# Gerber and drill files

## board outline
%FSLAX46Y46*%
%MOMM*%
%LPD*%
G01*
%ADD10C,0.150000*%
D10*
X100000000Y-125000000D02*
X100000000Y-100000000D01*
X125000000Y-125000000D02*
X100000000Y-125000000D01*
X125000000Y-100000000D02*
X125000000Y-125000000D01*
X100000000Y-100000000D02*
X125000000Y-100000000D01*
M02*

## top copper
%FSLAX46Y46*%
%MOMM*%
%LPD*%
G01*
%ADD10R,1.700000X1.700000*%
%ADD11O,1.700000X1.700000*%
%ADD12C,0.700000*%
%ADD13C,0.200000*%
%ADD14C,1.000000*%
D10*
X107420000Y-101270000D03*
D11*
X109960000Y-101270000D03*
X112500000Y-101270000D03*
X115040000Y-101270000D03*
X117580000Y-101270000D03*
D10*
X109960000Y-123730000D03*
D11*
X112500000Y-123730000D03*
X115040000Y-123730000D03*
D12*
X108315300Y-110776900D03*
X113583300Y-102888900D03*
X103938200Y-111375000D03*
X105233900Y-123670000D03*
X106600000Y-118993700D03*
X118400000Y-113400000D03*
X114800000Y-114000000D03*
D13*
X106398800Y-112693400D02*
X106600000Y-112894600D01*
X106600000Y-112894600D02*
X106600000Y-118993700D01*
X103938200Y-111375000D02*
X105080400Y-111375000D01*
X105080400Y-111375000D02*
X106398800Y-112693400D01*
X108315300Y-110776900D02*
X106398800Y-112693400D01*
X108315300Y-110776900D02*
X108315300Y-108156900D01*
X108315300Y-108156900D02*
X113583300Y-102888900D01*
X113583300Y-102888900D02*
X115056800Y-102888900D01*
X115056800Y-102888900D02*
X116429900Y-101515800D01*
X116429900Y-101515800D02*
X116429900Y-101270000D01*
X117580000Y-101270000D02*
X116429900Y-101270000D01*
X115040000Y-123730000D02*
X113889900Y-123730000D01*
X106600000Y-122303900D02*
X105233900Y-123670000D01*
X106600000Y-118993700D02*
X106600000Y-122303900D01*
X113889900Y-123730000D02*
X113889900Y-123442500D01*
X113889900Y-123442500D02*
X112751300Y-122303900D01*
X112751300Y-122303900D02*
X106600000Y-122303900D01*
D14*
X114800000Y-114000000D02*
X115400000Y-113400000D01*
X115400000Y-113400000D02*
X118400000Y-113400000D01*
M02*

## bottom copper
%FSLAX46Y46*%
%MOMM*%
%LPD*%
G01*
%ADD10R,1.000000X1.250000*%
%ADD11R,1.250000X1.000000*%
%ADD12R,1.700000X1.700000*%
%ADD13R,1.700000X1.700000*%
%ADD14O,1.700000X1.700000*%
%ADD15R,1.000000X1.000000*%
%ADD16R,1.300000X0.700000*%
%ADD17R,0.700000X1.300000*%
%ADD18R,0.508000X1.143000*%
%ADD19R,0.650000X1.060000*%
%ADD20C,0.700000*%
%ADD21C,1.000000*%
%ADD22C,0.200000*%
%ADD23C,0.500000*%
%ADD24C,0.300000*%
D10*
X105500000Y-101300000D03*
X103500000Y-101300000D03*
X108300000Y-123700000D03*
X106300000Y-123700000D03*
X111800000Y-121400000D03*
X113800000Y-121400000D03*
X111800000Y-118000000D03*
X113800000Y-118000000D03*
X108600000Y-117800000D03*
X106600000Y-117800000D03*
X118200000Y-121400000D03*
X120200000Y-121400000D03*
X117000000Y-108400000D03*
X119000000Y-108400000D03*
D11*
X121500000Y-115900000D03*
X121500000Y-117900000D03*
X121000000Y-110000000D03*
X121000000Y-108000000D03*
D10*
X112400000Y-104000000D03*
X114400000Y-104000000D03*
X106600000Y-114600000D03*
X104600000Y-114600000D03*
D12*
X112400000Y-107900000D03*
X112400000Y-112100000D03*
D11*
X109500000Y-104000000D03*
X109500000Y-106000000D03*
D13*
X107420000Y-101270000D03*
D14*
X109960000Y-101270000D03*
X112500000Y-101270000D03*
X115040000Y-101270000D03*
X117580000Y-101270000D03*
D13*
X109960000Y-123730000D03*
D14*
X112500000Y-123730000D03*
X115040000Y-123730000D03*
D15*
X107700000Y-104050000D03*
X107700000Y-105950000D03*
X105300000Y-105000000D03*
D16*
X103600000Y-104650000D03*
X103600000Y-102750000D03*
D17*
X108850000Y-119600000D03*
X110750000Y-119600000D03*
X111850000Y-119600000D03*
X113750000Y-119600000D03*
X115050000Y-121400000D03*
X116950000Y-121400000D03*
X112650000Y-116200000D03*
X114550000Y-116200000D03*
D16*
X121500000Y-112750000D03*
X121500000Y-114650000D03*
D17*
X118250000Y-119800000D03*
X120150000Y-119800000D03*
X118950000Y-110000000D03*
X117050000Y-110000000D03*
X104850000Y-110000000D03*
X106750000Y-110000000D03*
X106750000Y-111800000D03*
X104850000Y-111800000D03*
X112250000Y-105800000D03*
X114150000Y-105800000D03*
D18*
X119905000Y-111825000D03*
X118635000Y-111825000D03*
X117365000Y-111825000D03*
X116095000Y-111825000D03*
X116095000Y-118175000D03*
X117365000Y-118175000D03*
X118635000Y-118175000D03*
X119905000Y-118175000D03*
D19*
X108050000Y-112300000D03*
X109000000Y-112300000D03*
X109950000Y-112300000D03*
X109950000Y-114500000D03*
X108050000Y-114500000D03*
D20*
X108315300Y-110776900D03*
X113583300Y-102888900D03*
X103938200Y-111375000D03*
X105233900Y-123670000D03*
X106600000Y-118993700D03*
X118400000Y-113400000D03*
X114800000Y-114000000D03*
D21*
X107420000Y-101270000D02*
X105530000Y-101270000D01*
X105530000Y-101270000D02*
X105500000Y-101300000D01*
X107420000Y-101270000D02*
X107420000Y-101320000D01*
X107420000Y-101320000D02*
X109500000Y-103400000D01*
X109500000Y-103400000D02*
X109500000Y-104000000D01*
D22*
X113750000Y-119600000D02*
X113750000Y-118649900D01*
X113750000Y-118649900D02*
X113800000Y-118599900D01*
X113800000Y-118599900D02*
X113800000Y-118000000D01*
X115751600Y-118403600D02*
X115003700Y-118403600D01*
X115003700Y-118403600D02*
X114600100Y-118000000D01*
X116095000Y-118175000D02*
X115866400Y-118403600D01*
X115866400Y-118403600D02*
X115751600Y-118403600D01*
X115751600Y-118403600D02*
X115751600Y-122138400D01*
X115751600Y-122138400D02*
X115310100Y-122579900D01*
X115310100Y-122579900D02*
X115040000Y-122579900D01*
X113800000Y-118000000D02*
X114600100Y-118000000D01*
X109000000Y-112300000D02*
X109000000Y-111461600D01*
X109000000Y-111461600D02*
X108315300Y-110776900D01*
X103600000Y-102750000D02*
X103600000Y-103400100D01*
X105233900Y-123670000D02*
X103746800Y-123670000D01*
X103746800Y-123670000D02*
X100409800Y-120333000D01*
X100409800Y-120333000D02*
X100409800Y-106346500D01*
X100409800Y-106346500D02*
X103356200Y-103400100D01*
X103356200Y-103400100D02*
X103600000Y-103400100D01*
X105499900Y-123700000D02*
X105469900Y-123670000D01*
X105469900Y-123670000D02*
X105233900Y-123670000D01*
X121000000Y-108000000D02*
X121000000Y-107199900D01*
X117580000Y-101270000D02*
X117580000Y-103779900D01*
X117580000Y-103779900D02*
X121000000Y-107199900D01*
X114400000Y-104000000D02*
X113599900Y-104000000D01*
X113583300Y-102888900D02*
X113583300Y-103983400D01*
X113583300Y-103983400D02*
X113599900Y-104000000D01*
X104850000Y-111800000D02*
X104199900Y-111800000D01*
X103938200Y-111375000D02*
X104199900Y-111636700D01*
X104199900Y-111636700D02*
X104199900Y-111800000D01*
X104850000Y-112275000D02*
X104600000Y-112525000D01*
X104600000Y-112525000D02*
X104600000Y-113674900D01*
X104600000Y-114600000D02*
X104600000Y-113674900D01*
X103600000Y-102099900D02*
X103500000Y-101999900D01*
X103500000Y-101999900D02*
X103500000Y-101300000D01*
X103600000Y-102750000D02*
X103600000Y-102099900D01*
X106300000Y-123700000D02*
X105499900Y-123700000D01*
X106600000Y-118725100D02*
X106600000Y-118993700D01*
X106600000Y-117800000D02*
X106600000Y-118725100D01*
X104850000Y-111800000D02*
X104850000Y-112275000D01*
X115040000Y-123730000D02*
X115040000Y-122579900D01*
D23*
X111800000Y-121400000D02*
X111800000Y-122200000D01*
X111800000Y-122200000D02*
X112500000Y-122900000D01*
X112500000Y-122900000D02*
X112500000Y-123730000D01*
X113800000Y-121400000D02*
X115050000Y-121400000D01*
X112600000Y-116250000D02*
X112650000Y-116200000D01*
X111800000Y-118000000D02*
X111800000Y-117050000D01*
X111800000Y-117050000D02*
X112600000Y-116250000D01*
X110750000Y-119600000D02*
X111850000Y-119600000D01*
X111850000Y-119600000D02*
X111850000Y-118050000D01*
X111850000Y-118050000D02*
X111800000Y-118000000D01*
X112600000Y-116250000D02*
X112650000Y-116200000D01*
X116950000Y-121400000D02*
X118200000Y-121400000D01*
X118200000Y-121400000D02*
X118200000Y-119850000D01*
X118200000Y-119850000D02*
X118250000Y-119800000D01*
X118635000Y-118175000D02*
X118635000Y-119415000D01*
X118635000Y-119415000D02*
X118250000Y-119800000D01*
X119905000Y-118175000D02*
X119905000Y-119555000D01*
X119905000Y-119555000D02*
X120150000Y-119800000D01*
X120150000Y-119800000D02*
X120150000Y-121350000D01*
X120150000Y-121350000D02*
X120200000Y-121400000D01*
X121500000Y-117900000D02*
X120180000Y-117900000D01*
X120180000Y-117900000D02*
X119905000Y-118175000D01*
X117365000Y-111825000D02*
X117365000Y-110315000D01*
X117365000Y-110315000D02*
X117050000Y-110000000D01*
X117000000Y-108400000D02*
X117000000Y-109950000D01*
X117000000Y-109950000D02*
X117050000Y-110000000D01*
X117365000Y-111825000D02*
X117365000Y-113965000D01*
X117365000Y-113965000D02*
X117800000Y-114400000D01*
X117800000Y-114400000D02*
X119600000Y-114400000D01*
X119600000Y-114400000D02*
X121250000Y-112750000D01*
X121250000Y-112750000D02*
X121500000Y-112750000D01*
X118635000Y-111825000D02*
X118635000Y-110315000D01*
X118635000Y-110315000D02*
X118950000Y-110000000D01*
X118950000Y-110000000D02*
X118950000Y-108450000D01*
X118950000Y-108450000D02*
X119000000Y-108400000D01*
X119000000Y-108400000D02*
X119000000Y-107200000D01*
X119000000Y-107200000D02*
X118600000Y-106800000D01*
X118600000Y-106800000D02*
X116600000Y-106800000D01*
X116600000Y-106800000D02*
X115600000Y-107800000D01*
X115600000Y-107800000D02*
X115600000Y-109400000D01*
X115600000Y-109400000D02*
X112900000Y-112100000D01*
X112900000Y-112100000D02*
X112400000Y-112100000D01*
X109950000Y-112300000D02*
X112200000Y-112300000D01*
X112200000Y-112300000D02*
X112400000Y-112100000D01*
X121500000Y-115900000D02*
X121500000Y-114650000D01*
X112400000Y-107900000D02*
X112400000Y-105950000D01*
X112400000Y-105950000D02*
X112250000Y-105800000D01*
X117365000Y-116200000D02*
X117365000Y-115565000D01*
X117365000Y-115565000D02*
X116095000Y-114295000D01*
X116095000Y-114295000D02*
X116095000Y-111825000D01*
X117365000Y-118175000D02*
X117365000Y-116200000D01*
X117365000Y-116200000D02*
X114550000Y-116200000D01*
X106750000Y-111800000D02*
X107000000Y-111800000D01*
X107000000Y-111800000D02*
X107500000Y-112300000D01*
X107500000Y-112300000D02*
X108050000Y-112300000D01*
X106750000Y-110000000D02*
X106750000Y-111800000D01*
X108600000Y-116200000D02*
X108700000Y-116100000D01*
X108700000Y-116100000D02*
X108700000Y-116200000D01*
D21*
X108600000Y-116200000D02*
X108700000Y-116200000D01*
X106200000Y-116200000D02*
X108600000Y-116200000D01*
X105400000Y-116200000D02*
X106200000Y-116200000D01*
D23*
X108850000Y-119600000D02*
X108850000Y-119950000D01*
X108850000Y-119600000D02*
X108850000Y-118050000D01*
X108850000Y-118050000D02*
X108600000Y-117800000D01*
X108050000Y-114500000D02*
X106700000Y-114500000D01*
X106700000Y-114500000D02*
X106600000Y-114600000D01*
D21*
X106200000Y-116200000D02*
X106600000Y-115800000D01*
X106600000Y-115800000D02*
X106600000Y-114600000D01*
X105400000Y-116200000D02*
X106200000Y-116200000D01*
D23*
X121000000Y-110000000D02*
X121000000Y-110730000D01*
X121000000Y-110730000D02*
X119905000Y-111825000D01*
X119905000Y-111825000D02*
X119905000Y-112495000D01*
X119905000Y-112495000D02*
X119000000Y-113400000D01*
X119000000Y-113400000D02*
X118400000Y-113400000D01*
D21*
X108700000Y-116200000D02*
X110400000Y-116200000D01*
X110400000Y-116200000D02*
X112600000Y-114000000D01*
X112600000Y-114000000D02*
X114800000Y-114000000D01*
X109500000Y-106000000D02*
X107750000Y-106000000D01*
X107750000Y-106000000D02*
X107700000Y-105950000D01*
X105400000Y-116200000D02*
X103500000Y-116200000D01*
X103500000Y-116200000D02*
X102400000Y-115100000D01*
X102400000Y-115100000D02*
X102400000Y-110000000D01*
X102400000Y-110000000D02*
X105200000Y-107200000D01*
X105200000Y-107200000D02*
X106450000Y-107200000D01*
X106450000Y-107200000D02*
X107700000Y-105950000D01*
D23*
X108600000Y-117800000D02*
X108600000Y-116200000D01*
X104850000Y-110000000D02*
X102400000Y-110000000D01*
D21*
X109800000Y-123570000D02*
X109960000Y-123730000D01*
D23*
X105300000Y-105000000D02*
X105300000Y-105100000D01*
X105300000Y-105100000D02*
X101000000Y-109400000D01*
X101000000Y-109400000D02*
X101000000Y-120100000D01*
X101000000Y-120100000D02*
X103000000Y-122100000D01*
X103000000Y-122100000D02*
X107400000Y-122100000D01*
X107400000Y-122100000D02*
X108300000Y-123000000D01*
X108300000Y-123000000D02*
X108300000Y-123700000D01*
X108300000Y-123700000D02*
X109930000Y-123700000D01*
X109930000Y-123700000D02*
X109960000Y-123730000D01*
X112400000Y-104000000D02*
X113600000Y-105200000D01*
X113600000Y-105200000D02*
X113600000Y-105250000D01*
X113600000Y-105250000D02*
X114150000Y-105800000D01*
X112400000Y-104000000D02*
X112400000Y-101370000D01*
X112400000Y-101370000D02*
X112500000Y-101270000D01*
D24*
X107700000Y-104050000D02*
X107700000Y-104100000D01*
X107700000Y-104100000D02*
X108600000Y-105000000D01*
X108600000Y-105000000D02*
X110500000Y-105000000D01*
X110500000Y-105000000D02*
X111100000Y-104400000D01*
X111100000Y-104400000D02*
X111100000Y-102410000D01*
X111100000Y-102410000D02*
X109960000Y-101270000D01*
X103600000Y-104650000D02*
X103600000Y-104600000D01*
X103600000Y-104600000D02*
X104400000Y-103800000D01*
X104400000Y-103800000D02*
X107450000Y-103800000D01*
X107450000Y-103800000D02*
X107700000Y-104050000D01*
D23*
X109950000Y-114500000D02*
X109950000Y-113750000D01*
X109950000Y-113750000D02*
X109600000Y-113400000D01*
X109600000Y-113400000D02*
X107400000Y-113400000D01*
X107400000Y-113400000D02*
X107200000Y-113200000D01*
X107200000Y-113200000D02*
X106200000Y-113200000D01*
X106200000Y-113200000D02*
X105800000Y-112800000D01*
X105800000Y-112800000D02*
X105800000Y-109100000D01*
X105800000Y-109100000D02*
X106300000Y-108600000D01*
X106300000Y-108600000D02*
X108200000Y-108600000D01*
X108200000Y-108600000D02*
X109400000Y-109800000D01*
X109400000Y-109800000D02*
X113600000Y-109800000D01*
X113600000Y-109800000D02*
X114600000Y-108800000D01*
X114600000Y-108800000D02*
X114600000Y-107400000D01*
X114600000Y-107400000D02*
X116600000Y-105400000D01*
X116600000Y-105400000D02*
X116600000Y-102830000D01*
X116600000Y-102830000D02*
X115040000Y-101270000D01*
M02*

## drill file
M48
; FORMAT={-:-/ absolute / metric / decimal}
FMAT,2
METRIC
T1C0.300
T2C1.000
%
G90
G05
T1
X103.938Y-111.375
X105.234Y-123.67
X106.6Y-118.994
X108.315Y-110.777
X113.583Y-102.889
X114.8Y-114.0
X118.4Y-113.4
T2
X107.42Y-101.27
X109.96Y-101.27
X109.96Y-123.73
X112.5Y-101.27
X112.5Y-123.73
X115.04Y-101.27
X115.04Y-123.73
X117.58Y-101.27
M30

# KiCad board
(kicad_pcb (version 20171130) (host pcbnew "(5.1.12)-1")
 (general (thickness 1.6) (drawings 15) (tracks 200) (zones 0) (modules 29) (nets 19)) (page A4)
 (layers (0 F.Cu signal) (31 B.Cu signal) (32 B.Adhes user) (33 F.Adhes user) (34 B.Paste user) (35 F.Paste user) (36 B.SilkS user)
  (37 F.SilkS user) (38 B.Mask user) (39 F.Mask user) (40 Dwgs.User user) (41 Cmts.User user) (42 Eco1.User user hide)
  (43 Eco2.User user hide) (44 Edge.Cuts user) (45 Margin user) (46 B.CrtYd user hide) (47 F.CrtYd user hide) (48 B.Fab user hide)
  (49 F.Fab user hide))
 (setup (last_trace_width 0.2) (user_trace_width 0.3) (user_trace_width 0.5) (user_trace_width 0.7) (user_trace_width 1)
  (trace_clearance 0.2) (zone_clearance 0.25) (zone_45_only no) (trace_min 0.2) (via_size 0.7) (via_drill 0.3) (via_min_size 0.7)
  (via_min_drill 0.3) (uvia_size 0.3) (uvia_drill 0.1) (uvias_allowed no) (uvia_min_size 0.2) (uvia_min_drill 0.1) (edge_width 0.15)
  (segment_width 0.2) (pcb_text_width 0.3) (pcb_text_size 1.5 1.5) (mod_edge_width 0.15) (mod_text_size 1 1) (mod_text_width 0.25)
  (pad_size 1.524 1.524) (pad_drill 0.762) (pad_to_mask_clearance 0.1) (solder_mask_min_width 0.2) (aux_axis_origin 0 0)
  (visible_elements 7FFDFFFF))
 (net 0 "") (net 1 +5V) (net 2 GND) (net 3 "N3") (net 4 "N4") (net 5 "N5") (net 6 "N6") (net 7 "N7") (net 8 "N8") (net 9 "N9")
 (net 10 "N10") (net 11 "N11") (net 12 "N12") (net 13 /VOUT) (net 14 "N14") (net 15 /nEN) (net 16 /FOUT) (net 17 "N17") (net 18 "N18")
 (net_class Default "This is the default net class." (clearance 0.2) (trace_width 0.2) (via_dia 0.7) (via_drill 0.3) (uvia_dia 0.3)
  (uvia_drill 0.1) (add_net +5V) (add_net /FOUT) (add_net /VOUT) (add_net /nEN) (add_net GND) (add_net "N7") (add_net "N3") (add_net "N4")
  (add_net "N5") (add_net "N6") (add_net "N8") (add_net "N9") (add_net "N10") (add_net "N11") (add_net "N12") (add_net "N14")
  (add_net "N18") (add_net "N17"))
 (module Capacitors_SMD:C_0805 (layer B.Cu) (at 104.5 101.3 180)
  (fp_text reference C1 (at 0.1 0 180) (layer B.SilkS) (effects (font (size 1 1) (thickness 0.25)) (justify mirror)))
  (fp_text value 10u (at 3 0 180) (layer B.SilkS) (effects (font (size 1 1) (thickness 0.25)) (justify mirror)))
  (pad 1 smd rect (at -1 0 180) (size 1 1.25) (layers B.Cu B.Paste B.Mask) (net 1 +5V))
  (pad 2 smd rect (at 1 0 180) (size 1 1.25) (layers B.Cu B.Paste B.Mask) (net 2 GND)))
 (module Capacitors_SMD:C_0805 (layer B.Cu) (at 107.3 123.7 180)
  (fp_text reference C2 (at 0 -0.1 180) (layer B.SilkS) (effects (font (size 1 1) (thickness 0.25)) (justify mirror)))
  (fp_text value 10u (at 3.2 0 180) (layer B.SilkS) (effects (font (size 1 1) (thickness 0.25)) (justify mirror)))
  (pad 1 smd rect (at -1 0 180) (size 1 1.25) (layers B.Cu B.Paste B.Mask) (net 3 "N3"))
  (pad 2 smd rect (at 1 0 180) (size 1 1.25) (layers B.Cu B.Paste B.Mask) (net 2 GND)))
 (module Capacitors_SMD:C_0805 (layer B.Cu) (at 112.8 121.4)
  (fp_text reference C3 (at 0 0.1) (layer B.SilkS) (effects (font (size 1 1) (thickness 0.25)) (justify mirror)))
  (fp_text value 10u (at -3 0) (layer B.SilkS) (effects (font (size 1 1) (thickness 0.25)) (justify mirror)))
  (pad 1 smd rect (at -1 0) (size 1 1.25) (layers B.Cu B.Paste B.Mask) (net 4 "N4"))
  (pad 2 smd rect (at 1 0) (size 1 1.25) (layers B.Cu B.Paste B.Mask) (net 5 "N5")))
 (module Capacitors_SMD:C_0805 (layer B.Cu) (at 112.8 118)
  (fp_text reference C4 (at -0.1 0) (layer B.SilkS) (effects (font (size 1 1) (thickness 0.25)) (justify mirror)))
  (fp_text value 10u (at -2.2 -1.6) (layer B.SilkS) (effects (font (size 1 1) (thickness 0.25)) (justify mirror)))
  (pad 1 smd rect (at -1 0) (size 1 1.25) (layers B.Cu B.Paste B.Mask) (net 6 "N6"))
  (pad 2 smd rect (at 1 0) (size 1 1.25) (layers B.Cu B.Paste B.Mask) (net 2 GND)))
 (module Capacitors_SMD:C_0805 (layer B.Cu) (at 107.6 117.8 180)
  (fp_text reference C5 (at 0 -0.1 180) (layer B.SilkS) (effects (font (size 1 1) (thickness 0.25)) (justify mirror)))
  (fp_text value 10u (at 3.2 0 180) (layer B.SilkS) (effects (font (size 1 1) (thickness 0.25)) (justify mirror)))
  (pad 1 smd rect (at -1 0 180) (size 1 1.25) (layers B.Cu B.Paste B.Mask) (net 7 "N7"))
  (pad 2 smd rect (at 1 0 180) (size 1 1.25) (layers B.Cu B.Paste B.Mask) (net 2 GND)))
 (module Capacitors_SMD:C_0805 (layer B.Cu) (at 119.2 121.4)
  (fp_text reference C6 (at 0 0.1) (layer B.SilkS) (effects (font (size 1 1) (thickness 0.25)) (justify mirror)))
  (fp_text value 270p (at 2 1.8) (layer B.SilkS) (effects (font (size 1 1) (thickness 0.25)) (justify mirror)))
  (pad 1 smd rect (at -1 0) (size 1 1.25) (layers B.Cu B.Paste B.Mask) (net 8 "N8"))
  (pad 2 smd rect (at 1 0) (size 1 1.25) (layers B.Cu B.Paste B.Mask) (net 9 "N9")))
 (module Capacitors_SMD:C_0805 (layer B.Cu) (at 118 108.4)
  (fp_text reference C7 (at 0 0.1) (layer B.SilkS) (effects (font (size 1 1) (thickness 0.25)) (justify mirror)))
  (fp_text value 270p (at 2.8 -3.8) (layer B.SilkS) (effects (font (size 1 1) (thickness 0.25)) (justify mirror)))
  (pad 1 smd rect (at -1 0) (size 1 1.25) (layers B.Cu B.Paste B.Mask) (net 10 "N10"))
  (pad 2 smd rect (at 1 0) (size 1 1.25) (layers B.Cu B.Paste B.Mask) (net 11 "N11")))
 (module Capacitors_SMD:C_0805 (layer B.Cu) (at 121.5 116.9 270)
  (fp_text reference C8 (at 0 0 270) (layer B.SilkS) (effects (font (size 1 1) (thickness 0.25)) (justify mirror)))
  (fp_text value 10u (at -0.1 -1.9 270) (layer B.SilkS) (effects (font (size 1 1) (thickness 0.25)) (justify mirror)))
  (pad 1 smd rect (at -1 0 270) (size 1 1.25) (layers B.Cu B.Paste B.Mask) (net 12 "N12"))
  (pad 2 smd rect (at 1 0 270) (size 1 1.25) (layers B.Cu B.Paste B.Mask) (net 9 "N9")))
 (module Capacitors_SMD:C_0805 (layer B.Cu) (at 121 109 90)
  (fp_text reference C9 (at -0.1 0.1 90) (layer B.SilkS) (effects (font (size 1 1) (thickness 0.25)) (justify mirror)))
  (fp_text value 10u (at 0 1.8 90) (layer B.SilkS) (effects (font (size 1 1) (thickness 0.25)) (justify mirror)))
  (pad 1 smd rect (at -1 0 90) (size 1 1.25) (layers B.Cu B.Paste B.Mask) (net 7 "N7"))
  (pad 2 smd rect (at 1 0 90) (size 1 1.25) (layers B.Cu B.Paste B.Mask) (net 2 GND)))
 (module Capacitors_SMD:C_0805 (layer B.Cu) (at 113.4 104)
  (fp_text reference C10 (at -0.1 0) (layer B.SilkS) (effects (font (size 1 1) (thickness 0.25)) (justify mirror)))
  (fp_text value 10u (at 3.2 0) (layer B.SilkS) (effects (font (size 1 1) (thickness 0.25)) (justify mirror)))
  (pad 1 smd rect (at -1 0) (size 1 1.25) (layers B.Cu B.Paste B.Mask) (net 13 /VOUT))
  (pad 2 smd rect (at 1 0) (size 1 1.25) (layers B.Cu B.Paste B.Mask) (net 2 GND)))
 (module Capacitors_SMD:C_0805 (layer B.Cu) (at 105.6 114.6 180)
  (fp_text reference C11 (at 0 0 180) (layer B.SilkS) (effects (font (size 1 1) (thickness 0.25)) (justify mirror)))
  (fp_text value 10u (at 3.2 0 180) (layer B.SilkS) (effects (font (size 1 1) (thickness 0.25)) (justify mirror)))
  (pad 1 smd rect (at -1 0 180) (size 1 1.25) (layers B.Cu B.Paste B.Mask) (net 7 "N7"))
  (pad 2 smd rect (at 1 0 180) (size 1 1.25) (layers B.Cu B.Paste B.Mask) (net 2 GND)))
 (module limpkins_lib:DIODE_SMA (layer B.Cu) (at 112.4 110 270)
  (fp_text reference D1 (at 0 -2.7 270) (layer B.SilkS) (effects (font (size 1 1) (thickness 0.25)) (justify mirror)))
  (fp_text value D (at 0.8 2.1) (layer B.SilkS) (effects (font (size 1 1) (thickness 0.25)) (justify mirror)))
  (pad 1 smd rect (at -2.1 0 270) (size 1.7 1.7) (layers B.Cu B.Paste B.Mask) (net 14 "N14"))
  (pad 2 smd rect (at 2.1 0 270) (size 1.7 1.7) (layers B.Cu B.Paste B.Mask) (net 11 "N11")))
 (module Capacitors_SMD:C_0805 (layer B.Cu) (at 109.5 105 270)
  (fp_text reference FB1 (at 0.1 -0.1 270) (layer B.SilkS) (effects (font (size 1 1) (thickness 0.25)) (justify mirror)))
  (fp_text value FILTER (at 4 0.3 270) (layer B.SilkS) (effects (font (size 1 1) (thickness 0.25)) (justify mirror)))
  (pad 1 smd rect (at -1 0 270) (size 1 1.25) (layers B.Cu B.Paste B.Mask) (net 1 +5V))
  (pad 2 smd rect (at 1 0 270) (size 1 1.25) (layers B.Cu B.Paste B.Mask) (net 7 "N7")))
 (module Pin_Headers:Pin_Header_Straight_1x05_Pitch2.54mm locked (layer F.Cu) (at 107.42 101.27 90)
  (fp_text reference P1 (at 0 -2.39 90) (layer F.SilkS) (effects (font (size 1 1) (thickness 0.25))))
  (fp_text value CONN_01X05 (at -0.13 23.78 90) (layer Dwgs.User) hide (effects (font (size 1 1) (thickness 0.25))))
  (pad 1 thru_hole rect (at 0 0 90) (size 1.7 1.7) (drill 1) (layers *.Cu *.Mask) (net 1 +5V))
  (pad 2 thru_hole oval (at 0 2.54 90) (size 1.7 1.7) (drill 1) (layers *.Cu *.Mask) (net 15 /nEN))
  (pad 3 thru_hole oval (at 0 5.08 90) (size 1.7 1.7) (drill 1) (layers *.Cu *.Mask) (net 13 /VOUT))
  (pad 4 thru_hole oval (at 0 7.62 90) (size 1.7 1.7) (drill 1) (layers *.Cu *.Mask) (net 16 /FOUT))
  (pad 5 thru_hole oval (at 0 10.16 90) (size 1.7 1.7) (drill 1) (layers *.Cu *.Mask) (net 2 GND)))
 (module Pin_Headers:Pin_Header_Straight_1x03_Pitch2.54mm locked (layer F.Cu) (at 109.96 123.73 90)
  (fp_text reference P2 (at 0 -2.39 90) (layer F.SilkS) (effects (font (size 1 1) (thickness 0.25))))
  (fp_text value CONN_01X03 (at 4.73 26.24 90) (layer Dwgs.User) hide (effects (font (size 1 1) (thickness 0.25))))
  (pad 1 thru_hole rect (at 0 0 90) (size 1.7 1.7) (drill 1) (layers *.Cu *.Mask) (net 3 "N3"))
  (pad 2 thru_hole oval (at 0 2.54 90) (size 1.7 1.7) (drill 1) (layers *.Cu *.Mask) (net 4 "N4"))
  (pad 3 thru_hole oval (at 0 5.08 90) (size 1.7 1.7) (drill 1) (layers *.Cu *.Mask) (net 2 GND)))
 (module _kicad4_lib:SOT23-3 (layer B.Cu) (at 106.5 105 270)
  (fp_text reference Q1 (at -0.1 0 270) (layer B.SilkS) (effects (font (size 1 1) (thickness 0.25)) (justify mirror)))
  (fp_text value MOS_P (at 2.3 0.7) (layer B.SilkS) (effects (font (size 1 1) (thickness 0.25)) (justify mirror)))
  (pad 1 smd rect (at -0.95 -1.2 270) (size 1 1) (layers B.Cu B.Paste B.Mask) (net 15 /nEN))
  (pad 2 smd rect (at 0.95 -1.2 270) (size 1 1) (layers B.Cu B.Paste B.Mask) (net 7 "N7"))
  (pad 3 smd rect (at 0 1.2 270) (size 1 1) (layers B.Cu B.Paste B.Mask) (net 3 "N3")))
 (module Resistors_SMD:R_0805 (layer B.Cu) (at 103.6 103.7 90)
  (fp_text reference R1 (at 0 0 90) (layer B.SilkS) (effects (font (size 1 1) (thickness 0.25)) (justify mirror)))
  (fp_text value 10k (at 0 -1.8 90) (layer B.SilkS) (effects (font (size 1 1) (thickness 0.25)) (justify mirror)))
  (pad 1 smd rect (at -0.95 0 90) (size 0.7 1.3) (layers B.Cu B.Paste B.Mask) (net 15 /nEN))
  (pad 2 smd rect (at 0.95 0 90) (size 0.7 1.3) (layers B.Cu B.Paste B.Mask) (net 2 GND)))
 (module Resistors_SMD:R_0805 (layer B.Cu) (at 109.8 119.6)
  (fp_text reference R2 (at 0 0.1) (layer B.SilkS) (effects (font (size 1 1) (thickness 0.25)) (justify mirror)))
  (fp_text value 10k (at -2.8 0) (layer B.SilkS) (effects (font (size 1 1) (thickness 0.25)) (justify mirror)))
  (pad 1 smd rect (at -0.95 0) (size 0.7 1.3) (layers B.Cu B.Paste B.Mask) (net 7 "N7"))
  (pad 2 smd rect (at 0.95 0) (size 0.7 1.3) (layers B.Cu B.Paste B.Mask) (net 6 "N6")))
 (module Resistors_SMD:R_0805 (layer B.Cu) (at 112.8 119.6)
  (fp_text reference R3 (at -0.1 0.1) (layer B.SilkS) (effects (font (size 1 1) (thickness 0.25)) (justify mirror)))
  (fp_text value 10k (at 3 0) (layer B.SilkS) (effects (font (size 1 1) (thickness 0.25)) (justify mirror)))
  (pad 1 smd rect (at -0.95 0) (size 0.7 1.3) (layers B.Cu B.Paste B.Mask) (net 6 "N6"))
  (pad 2 smd rect (at 0.95 0) (size 0.7 1.3) (layers B.Cu B.Paste B.Mask) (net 2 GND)))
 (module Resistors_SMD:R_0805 (layer B.Cu) (at 116 121.4)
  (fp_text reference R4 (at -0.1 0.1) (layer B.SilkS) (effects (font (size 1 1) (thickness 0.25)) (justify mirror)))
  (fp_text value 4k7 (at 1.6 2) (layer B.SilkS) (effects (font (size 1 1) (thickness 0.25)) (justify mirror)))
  (pad 1 smd rect (at -0.95 0) (size 0.7 1.3) (layers B.Cu B.Paste B.Mask) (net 5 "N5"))
  (pad 2 smd rect (at 0.95 0) (size 0.7 1.3) (layers B.Cu B.Paste B.Mask) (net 8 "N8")))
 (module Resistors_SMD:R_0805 (layer B.Cu) (at 113.6 116.2)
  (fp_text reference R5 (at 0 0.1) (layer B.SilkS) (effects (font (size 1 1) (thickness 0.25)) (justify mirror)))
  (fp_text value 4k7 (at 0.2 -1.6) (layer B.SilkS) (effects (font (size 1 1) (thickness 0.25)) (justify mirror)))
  (pad 1 smd rect (at -0.95 0) (size 0.7 1.3) (layers B.Cu B.Paste B.Mask) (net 6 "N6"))
  (pad 2 smd rect (at 0.95 0) (size 0.7 1.3) (layers B.Cu B.Paste B.Mask) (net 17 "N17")))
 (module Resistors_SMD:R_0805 (layer B.Cu) (at 121.5 113.7 270)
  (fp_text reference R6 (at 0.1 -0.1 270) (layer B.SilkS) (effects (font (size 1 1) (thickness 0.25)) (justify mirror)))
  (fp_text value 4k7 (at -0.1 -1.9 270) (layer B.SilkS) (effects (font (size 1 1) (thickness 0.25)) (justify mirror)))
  (pad 1 smd rect (at -0.95 0 270) (size 0.7 1.3) (layers B.Cu B.Paste B.Mask) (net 10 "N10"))
  (pad 2 smd rect (at 0.95 0 270) (size 0.7 1.3) (layers B.Cu B.Paste B.Mask) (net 12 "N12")))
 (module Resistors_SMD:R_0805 (layer B.Cu) (at 119.2 119.8)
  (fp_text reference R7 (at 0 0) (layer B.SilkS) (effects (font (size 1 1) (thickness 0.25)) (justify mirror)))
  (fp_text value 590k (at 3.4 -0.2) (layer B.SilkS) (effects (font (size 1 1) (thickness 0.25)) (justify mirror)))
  (pad 1 smd rect (at -0.95 0) (size 0.7 1.3) (layers B.Cu B.Paste B.Mask) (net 8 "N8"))
  (pad 2 smd rect (at 0.95 0) (size 0.7 1.3) (layers B.Cu B.Paste B.Mask) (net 9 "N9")))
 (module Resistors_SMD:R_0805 (layer B.Cu) (at 118 110 180)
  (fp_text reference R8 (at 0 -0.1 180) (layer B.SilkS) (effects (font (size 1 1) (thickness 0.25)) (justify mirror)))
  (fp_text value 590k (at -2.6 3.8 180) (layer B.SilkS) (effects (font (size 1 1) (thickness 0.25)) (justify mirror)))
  (pad 1 smd rect (at -0.95 0 180) (size 0.7 1.3) (layers B.Cu B.Paste B.Mask) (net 11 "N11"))
  (pad 2 smd rect (at 0.95 0 180) (size 0.7 1.3) (layers B.Cu B.Paste B.Mask) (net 10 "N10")))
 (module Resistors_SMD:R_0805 (layer B.Cu) (at 105.8 110)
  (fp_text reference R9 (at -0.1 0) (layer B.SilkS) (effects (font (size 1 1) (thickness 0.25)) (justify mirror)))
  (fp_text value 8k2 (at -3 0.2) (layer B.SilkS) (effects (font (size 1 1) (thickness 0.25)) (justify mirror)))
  (pad 1 smd rect (at -0.95 0) (size 0.7 1.3) (layers B.Cu B.Paste B.Mask) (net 7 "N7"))
  (pad 2 smd rect (at 0.95 0) (size 0.7 1.3) (layers B.Cu B.Paste B.Mask) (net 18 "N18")))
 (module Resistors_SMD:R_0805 (layer B.Cu) (at 105.8 111.8 180)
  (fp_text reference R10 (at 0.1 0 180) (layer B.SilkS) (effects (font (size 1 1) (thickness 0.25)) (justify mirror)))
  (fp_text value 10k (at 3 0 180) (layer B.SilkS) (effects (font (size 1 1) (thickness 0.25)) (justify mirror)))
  (pad 1 smd rect (at -0.95 0 180) (size 0.7 1.3) (layers B.Cu B.Paste B.Mask) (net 18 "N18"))
  (pad 2 smd rect (at 0.95 0 180) (size 0.7 1.3) (layers B.Cu B.Paste B.Mask) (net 2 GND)))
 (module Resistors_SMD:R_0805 (layer B.Cu) (at 113.2 105.8)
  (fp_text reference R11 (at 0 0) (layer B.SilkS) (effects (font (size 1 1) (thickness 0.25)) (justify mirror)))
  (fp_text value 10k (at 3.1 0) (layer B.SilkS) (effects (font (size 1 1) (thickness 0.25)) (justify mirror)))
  (pad 1 smd rect (at -0.95 0) (size 0.7 1.3) (layers B.Cu B.Paste B.Mask) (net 14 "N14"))
  (pad 2 smd rect (at 0.95 0) (size 0.7 1.3) (layers B.Cu B.Paste B.Mask) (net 13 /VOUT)))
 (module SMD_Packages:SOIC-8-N (layer B.Cu) (at 118 115 180)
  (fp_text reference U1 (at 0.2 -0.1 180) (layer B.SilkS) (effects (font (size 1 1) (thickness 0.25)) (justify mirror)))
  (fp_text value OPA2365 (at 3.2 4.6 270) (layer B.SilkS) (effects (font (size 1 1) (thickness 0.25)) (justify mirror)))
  (pad 8 smd rect (at -1.905 3.175 180) (size 0.508 1.143) (layers B.Cu B.Paste B.Mask) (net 7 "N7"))
  (pad 7 smd rect (at -0.635 3.175 180) (size 0.508 1.143) (layers B.Cu B.Paste B.Mask) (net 11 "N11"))
  (pad 6 smd rect (at 0.635 3.175 180) (size 0.508 1.143) (layers B.Cu B.Paste B.Mask) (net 10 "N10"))
  (pad 5 smd rect (at 1.905 3.175 180) (size 0.508 1.143) (layers B.Cu B.Paste B.Mask) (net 17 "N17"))
  (pad 4 smd rect (at 1.905 -3.175 180) (size 0.508 1.143) (layers B.Cu B.Paste B.Mask) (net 2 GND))
  (pad 3 smd rect (at 0.635 -3.175 180) (size 0.508 1.143) (layers B.Cu B.Paste B.Mask) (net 17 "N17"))
  (pad 2 smd rect (at -0.635 -3.175 180) (size 0.508 1.143) (layers B.Cu B.Paste B.Mask) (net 8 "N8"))
  (pad 1 smd rect (at -1.905 -3.175 180) (size 0.508 1.143) (layers B.Cu B.Paste B.Mask) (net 9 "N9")))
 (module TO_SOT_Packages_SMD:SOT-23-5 (layer B.Cu) (at 109 113.4 270)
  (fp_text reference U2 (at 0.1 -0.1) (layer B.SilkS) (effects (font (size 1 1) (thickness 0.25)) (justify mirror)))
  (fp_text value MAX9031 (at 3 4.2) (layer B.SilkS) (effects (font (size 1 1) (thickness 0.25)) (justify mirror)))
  (pad 1 smd rect (at -1.1 0.95 270) (size 1.06 0.65) (layers B.Cu B.Paste B.Mask) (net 18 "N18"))
  (pad 2 smd rect (at -1.1 0 270) (size 1.06 0.65) (layers B.Cu B.Paste B.Mask) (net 2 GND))
  (pad 3 smd rect (at -1.1 -0.95 270) (size 1.06 0.65) (layers B.Cu B.Paste B.Mask) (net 11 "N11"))
  (pad 4 smd rect (at 1.1 -0.95 270) (size 1.06 0.65) (layers B.Cu B.Paste B.Mask) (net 16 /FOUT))
  (pad 5 smd rect (at 1.1 0.95 270) (size 1.06 0.65) (layers B.Cu B.Paste B.Mask) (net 7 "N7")))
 (gr_line (start 100 125) (end 100 100) (angle 90) (layer Edge.Cuts) (width 0.15))
 (gr_line (start 125 125) (end 100 125) (angle 90) (layer Edge.Cuts) (width 0.15))
 (gr_line (start 125 100) (end 125 125) (angle 90) (layer Edge.Cuts) (width 0.15))
 (gr_line (start 100 100) (end 125 100) (angle 90) (layer Edge.Cuts) (width 0.15))
 (segment (start 107.42 101.27) (end 105.53 101.27) (width 1) (layer B.Cu) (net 1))
 (segment (start 105.53 101.27) (end 105.5 101.3) (width 1) (layer B.Cu) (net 1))
 (segment (start 107.42 101.27) (end 107.42 101.32) (width 1) (layer B.Cu) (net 1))
 (segment (start 107.42 101.32) (end 109.5 103.4) (width 1) (layer B.Cu) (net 1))
 (segment (start 109.5 103.4) (end 109.5 104) (width 1) (layer B.Cu) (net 1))
 (segment (start 113.75 119.6) (end 113.75 118.6499) (width 0.2) (layer B.Cu) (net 2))
 (segment (start 113.75 118.6499) (end 113.8 118.5999) (width 0.2) (layer B.Cu) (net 2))
 (segment (start 113.8 118.5999) (end 113.8 118) (width 0.2) (layer B.Cu) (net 2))
 (segment (start 115.7516 118.4036) (end 115.0037 118.4036) (width 0.2) (layer B.Cu) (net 2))
 (segment (start 115.0037 118.4036) (end 114.6001 118) (width 0.2) (layer B.Cu) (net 2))
 (segment (start 116.095 118.175) (end 115.8664 118.4036) (width 0.2) (layer B.Cu) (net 2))
 (segment (start 115.8664 118.4036) (end 115.7516 118.4036) (width 0.2) (layer B.Cu) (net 2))
 (segment (start 115.7516 118.4036) (end 115.7516 122.1384) (width 0.2) (layer B.Cu) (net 2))
 (segment (start 115.7516 122.1384) (end 115.3101 122.5799) (width 0.2) (layer B.Cu) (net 2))
 (segment (start 115.3101 122.5799) (end 115.04 122.5799) (width 0.2) (layer B.Cu) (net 2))
 (segment (start 113.8 118) (end 114.6001 118) (width 0.2) (layer B.Cu) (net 2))
 (segment (start 109 112.3) (end 109 111.4616) (width 0.2) (layer B.Cu) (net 2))
 (segment (start 109 111.4616) (end 108.3153 110.7769) (width 0.2) (layer B.Cu) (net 2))
 (segment (start 106.3988 112.6934) (end 106.6 112.8946) (width 0.2) (layer F.Cu) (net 2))
 (segment (start 106.6 112.8946) (end 106.6 118.9937) (width 0.2) (layer F.Cu) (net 2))
 (segment (start 103.9382 111.375) (end 105.0804 111.375) (width 0.2) (layer F.Cu) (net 2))
 (segment (start 105.0804 111.375) (end 106.3988 112.6934) (width 0.2) (layer F.Cu) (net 2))
 (segment (start 108.3153 110.7769) (end 106.3988 112.6934) (width 0.2) (layer F.Cu) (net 2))
 (segment (start 108.3153 110.7769) (end 108.3153 108.1569) (width 0.2) (layer F.Cu) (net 2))
 (segment (start 108.3153 108.1569) (end 113.5833 102.8889) (width 0.2) (layer F.Cu) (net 2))
 (segment (start 103.6 102.75) (end 103.6 103.4001) (width 0.2) (layer B.Cu) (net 2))
 (segment (start 105.2339 123.67) (end 103.7468 123.67) (width 0.2) (layer B.Cu) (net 2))
 (segment (start 103.7468 123.67) (end 100.4098 120.333) (width 0.2) (layer B.Cu) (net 2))
 (segment (start 100.4098 120.333) (end 100.4098 106.3465) (width 0.2) (layer B.Cu) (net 2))
 (segment (start 100.4098 106.3465) (end 103.3562 103.4001) (width 0.2) (layer B.Cu) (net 2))
 (segment (start 103.3562 103.4001) (end 103.6 103.4001) (width 0.2) (layer B.Cu) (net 2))
 (segment (start 105.4999 123.7) (end 105.4699 123.67) (width 0.2) (layer B.Cu) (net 2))
 (segment (start 105.4699 123.67) (end 105.2339 123.67) (width 0.2) (layer B.Cu) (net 2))
 (segment (start 121 108) (end 121 107.1999) (width 0.2) (layer B.Cu) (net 2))
 (segment (start 117.58 101.27) (end 117.58 103.7799) (width 0.2) (layer B.Cu) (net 2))
 (segment (start 117.58 103.7799) (end 121 107.1999) (width 0.2) (layer B.Cu) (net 2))
 (segment (start 113.5833 102.8889) (end 115.0568 102.8889) (width 0.2) (layer F.Cu) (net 2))
 (segment (start 115.0568 102.8889) (end 116.4299 101.5158) (width 0.2) (layer F.Cu) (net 2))
 (segment (start 116.4299 101.5158) (end 116.4299 101.27) (width 0.2) (layer F.Cu) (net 2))
 (segment (start 114.4 104) (end 113.5999 104) (width 0.2) (layer B.Cu) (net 2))
 (segment (start 113.5833 102.8889) (end 113.5833 103.9834) (width 0.2) (layer B.Cu) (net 2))
 (segment (start 113.5833 103.9834) (end 113.5999 104) (width 0.2) (layer B.Cu) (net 2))
 (segment (start 117.58 101.27) (end 116.4299 101.27) (width 0.2) (layer F.Cu) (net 2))
 (segment (start 104.85 111.8) (end 104.1999 111.8) (width 0.2) (layer B.Cu) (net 2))
 (segment (start 103.9382 111.375) (end 104.1999 111.6367) (width 0.2) (layer B.Cu) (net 2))
 (segment (start 104.1999 111.6367) (end 104.1999 111.8) (width 0.2) (layer B.Cu) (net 2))
 (segment (start 104.85 112.275) (end 104.6 112.525) (width 0.2) (layer B.Cu) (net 2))
 (segment (start 104.6 112.525) (end 104.6 113.6749) (width 0.2) (layer B.Cu) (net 2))
 (segment (start 115.04 123.73) (end 113.8899 123.73) (width 0.2) (layer F.Cu) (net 2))
 (segment (start 106.6 122.3039) (end 105.2339 123.67) (width 0.2) (layer F.Cu) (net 2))
 (segment (start 106.6 118.9937) (end 106.6 122.3039) (width 0.2) (layer F.Cu) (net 2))
 (segment (start 113.8899 123.73) (end 113.8899 123.4425) (width 0.2) (layer F.Cu) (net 2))
 (segment (start 113.8899 123.4425) (end 112.7513 122.3039) (width 0.2) (layer F.Cu) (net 2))
 (segment (start 112.7513 122.3039) (end 106.6 122.3039) (width 0.2) (layer F.Cu) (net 2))
 (segment (start 104.6 114.6) (end 104.6 113.6749) (width 0.2) (layer B.Cu) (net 2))
 (segment (start 103.6 102.0999) (end 103.5 101.9999) (width 0.2) (layer B.Cu) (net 2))
 (segment (start 103.5 101.9999) (end 103.5 101.3) (width 0.2) (layer B.Cu) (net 2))
 (segment (start 103.6 102.75) (end 103.6 102.0999) (width 0.2) (layer B.Cu) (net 2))
 (segment (start 106.3 123.7) (end 105.4999 123.7) (width 0.2) (layer B.Cu) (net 2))
 (segment (start 106.6 118.7251) (end 106.6 118.9937) (width 0.2) (layer B.Cu) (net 2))
 (segment (start 106.6 117.8) (end 106.6 118.7251) (width 0.2) (layer B.Cu) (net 2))
 (segment (start 104.85 111.8) (end 104.85 112.275) (width 0.2) (layer B.Cu) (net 2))
 (segment (start 115.04 123.73) (end 115.04 122.5799) (width 0.2) (layer B.Cu) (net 2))
 (via (at 108.3153 110.7769) (size 0.7) (layers F.Cu B.Cu) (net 2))
 (via (at 113.5833 102.8889) (size 0.7) (layers F.Cu B.Cu) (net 2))
 (via (at 103.9382 111.375) (size 0.7) (layers F.Cu B.Cu) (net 2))
 (via (at 105.2339 123.67) (size 0.7) (layers F.Cu B.Cu) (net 2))
 (via (at 106.6 118.9937) (size 0.7) (layers F.Cu B.Cu) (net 2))
 (segment (start 111.8 121.4) (end 111.8 122.2) (width 0.5) (layer B.Cu) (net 4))
 (segment (start 111.8 122.2) (end 112.5 122.9) (width 0.5) (layer B.Cu) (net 4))
 (segment (start 112.5 122.9) (end 112.5 123.73) (width 0.5) (layer B.Cu) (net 4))
 (segment (start 113.8 121.4) (end 115.05 121.4) (width 0.5) (layer B.Cu) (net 5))
 (segment (start 112.6 116.25) (end 112.65 116.2) (width 0.5) (layer B.Cu) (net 6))
 (segment (start 111.8 118) (end 111.8 117.05) (width 0.5) (layer B.Cu) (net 6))
 (segment (start 111.8 117.05) (end 112.6 116.25) (width 0.5) (layer B.Cu) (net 6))
 (segment (start 110.75 119.6) (end 111.85 119.6) (width 0.5) (layer B.Cu) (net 6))
 (segment (start 111.85 119.6) (end 111.85 118.05) (width 0.5) (layer B.Cu) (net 6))
 (segment (start 111.85 118.05) (end 111.8 118) (width 0.5) (layer B.Cu) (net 6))
 (segment (start 112.6 116.25) (end 112.65 116.2) (width 0.5) (layer B.Cu) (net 6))
 (segment (start 116.95 121.4) (end 118.2 121.4) (width 0.5) (layer B.Cu) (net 8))
 (segment (start 118.2 121.4) (end 118.2 119.85) (width 0.5) (layer B.Cu) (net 8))
 (segment (start 118.2 119.85) (end 118.25 119.8) (width 0.5) (layer B.Cu) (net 8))
 (segment (start 118.635 118.175) (end 118.635 119.415) (width 0.5) (layer B.Cu) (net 8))
 (segment (start 118.635 119.415) (end 118.25 119.8) (width 0.5) (layer B.Cu) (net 8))
 (segment (start 119.905 118.175) (end 119.905 119.555) (width 0.5) (layer B.Cu) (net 9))
 (segment (start 119.905 119.555) (end 120.15 119.8) (width 0.5) (layer B.Cu) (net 9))
 (segment (start 120.15 119.8) (end 120.15 121.35) (width 0.5) (layer B.Cu) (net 9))
 (segment (start 120.15 121.35) (end 120.2 121.4) (width 0.5) (layer B.Cu) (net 9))
 (segment (start 121.5 117.9) (end 120.18 117.9) (width 0.5) (layer B.Cu) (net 9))
 (segment (start 120.18 117.9) (end 119.905 118.175) (width 0.5) (layer B.Cu) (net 9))
 (segment (start 117.365 111.825) (end 117.365 110.315) (width 0.5) (layer B.Cu) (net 10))
 (segment (start 117.365 110.315) (end 117.05 110) (width 0.5) (layer B.Cu) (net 10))
 (segment (start 117 108.4) (end 117 109.95) (width 0.5) (layer B.Cu) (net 10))
 (segment (start 117 109.95) (end 117.05 110) (width 0.5) (layer B.Cu) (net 10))
 (segment (start 117.365 111.825) (end 117.365 113.965) (width 0.5) (layer B.Cu) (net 10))
 (segment (start 117.365 113.965) (end 117.8 114.4) (width 0.5) (layer B.Cu) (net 10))
 (segment (start 117.8 114.4) (end 119.6 114.4) (width 0.5) (layer B.Cu) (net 10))
 (segment (start 119.6 114.4) (end 121.25 112.75) (width 0.5) (layer B.Cu) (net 10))
 (segment (start 121.25 112.75) (end 121.5 112.75) (width 0.5) (layer B.Cu) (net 10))
 (segment (start 118.635 111.825) (end 118.635 110.315) (width 0.5) (layer B.Cu) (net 11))
 (segment (start 118.635 110.315) (end 118.95 110) (width 0.5) (layer B.Cu) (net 11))
 (segment (start 118.95 110) (end 118.95 108.45) (width 0.5) (layer B.Cu) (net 11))
 (segment (start 118.95 108.45) (end 119 108.4) (width 0.5) (layer B.Cu) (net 11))
 (segment (start 119 108.4) (end 119 107.2) (width 0.5) (layer B.Cu) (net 11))
 (segment (start 119 107.2) (end 118.6 106.8) (width 0.5) (layer B.Cu) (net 11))
 (segment (start 118.6 106.8) (end 116.6 106.8) (width 0.5) (layer B.Cu) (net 11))
 (segment (start 116.6 106.8) (end 115.6 107.8) (width 0.5) (layer B.Cu) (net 11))
 (segment (start 115.6 107.8) (end 115.6 109.4) (width 0.5) (layer B.Cu) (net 11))
 (segment (start 115.6 109.4) (end 112.9 112.1) (width 0.5) (layer B.Cu) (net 11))
 (segment (start 112.9 112.1) (end 112.4 112.1) (width 0.5) (layer B.Cu) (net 11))
 (segment (start 109.95 112.3) (end 112.2 112.3) (width 0.5) (layer B.Cu) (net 11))
 (segment (start 112.2 112.3) (end 112.4 112.1) (width 0.5) (layer B.Cu) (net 11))
 (segment (start 121.5 115.9) (end 121.5 114.65) (width 0.5) (layer B.Cu) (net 12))
 (segment (start 112.4 107.9) (end 112.4 105.95) (width 0.5) (layer B.Cu) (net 14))
 (segment (start 112.4 105.95) (end 112.25 105.8) (width 0.5) (layer B.Cu) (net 14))
 (segment (start 117.365 116.2) (end 117.365 115.565) (width 0.5) (layer B.Cu) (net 17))
 (segment (start 117.365 115.565) (end 116.095 114.295) (width 0.5) (layer B.Cu) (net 17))
 (segment (start 116.095 114.295) (end 116.095 111.825) (width 0.5) (layer B.Cu) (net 17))
 (segment (start 117.365 118.175) (end 117.365 116.2) (width 0.5) (layer B.Cu) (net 17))
 (segment (start 117.365 116.2) (end 114.55 116.2) (width 0.5) (layer B.Cu) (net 17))
 (segment (start 106.75 111.8) (end 107 111.8) (width 0.5) (layer B.Cu) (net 18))
 (segment (start 107 111.8) (end 107.5 112.3) (width 0.5) (layer B.Cu) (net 18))
 (segment (start 107.5 112.3) (end 108.05 112.3) (width 0.5) (layer B.Cu) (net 18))
 (segment (start 106.75 110) (end 106.75 111.8) (width 0.5) (layer B.Cu) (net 18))
 (segment (start 108.6 116.2) (end 108.7 116.1) (width 0.5) (layer B.Cu) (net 7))
 (segment (start 108.7 116.1) (end 108.7 116.2) (width 0.5) (layer B.Cu) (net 7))
 (segment (start 108.6 116.2) (end 108.7 116.2) (width 1) (layer B.Cu) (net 7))
 (segment (start 106.2 116.2) (end 108.6 116.2) (width 1) (layer B.Cu) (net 7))
 (segment (start 105.4 116.2) (end 106.2 116.2) (width 1) (layer B.Cu) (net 7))
 (segment (start 108.85 119.6) (end 108.85 119.95) (width 0.5) (layer B.Cu) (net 7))
 (segment (start 108.85 119.6) (end 108.85 118.05) (width 0.5) (layer B.Cu) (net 7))
 (segment (start 108.85 118.05) (end 108.6 117.8) (width 0.5) (layer B.Cu) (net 7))
 (segment (start 108.05 114.5) (end 106.7 114.5) (width 0.5) (layer B.Cu) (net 7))
 (segment (start 106.7 114.5) (end 106.6 114.6) (width 0.5) (layer B.Cu) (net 7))
 (segment (start 106.2 116.2) (end 106.6 115.8) (width 1) (layer B.Cu) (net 7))
 (segment (start 106.6 115.8) (end 106.6 114.6) (width 1) (layer B.Cu) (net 7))
 (segment (start 105.4 116.2) (end 106.2 116.2) (width 1) (layer B.Cu) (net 7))
 (segment (start 121 110) (end 121 110.73) (width 0.5) (layer B.Cu) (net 7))
 (segment (start 121 110.73) (end 119.905 111.825) (width 0.5) (layer B.Cu) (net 7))
 (segment (start 119.905 111.825) (end 119.905 112.495) (width 0.5) (layer B.Cu) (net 7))
 (segment (start 119.905 112.495) (end 119 113.4) (width 0.5) (layer B.Cu) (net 7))
 (segment (start 119 113.4) (end 118.4 113.4) (width 0.5) (layer B.Cu) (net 7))
 (segment (start 114.8 114) (end 115.4 113.4) (width 1) (layer F.Cu) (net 7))
 (segment (start 115.4 113.4) (end 118.4 113.4) (width 1) (layer F.Cu) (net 7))
 (segment (start 108.7 116.2) (end 110.4 116.2) (width 1) (layer B.Cu) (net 7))
 (segment (start 110.4 116.2) (end 112.6 114) (width 1) (layer B.Cu) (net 7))
 (segment (start 112.6 114) (end 114.8 114) (width 1) (layer B.Cu) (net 7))
 (segment (start 109.5 106) (end 107.75 106) (width 1) (layer B.Cu) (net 7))
 (segment (start 107.75 106) (end 107.7 105.95) (width 1) (layer B.Cu) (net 7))
 (segment (start 105.4 116.2) (end 103.5 116.2) (width 1) (layer B.Cu) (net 7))
 (segment (start 103.5 116.2) (end 102.4 115.1) (width 1) (layer B.Cu) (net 7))
 (segment (start 102.4 115.1) (end 102.4 110) (width 1) (layer B.Cu) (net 7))
 (segment (start 102.4 110) (end 105.2 107.2) (width 1) (layer B.Cu) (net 7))
 (segment (start 105.2 107.2) (end 106.45 107.2) (width 1) (layer B.Cu) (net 7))
 (segment (start 106.45 107.2) (end 107.7 105.95) (width 1) (layer B.Cu) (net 7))
 (segment (start 108.6 117.8) (end 108.6 116.2) (width 0.5) (layer B.Cu) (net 7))
 (segment (start 104.85 110) (end 102.4 110) (width 0.5) (layer B.Cu) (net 7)) (via (at 118.4 113.4) (size 0.7) (layers F.Cu B.Cu) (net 7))
 (via (at 114.8 114) (size 0.7) (layers F.Cu B.Cu) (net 7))
 (segment (start 109.8 123.57) (end 109.96 123.73) (width 1) (layer B.Cu) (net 3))
 (segment (start 105.3 105) (end 105.3 105.1) (width 0.5) (layer B.Cu) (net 3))
 (segment (start 105.3 105.1) (end 101 109.4) (width 0.5) (layer B.Cu) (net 3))
 (segment (start 101 109.4) (end 101 120.1) (width 0.5) (layer B.Cu) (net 3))
 (segment (start 101 120.1) (end 103 122.1) (width 0.5) (layer B.Cu) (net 3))
 (segment (start 103 122.1) (end 107.4 122.1) (width 0.5) (layer B.Cu) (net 3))
 (segment (start 107.4 122.1) (end 108.3 123) (width 0.5) (layer B.Cu) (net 3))
 (segment (start 108.3 123) (end 108.3 123.7) (width 0.5) (layer B.Cu) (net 3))
 (segment (start 108.3 123.7) (end 109.93 123.7) (width 0.5) (layer B.Cu) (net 3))
 (segment (start 109.93 123.7) (end 109.96 123.73) (width 0.5) (layer B.Cu) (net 3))
 (segment (start 112.4 104) (end 113.6 105.2) (width 0.5) (layer B.Cu) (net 13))
 (segment (start 113.6 105.2) (end 113.6 105.25) (width 0.5) (layer B.Cu) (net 13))
 (segment (start 113.6 105.25) (end 114.15 105.8) (width 0.5) (layer B.Cu) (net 13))
 (segment (start 112.4 104) (end 112.4 101.37) (width 0.5) (layer B.Cu) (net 13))
 (segment (start 112.4 101.37) (end 112.5 101.27) (width 0.5) (layer B.Cu) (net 13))
 (segment (start 107.7 104.05) (end 107.7 104.1) (width 0.3) (layer B.Cu) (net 15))
 (segment (start 107.7 104.1) (end 108.6 105) (width 0.3) (layer B.Cu) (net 15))
 (segment (start 108.6 105) (end 110.5 105) (width 0.3) (layer B.Cu) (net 15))
 (segment (start 110.5 105) (end 111.1 104.4) (width 0.3) (layer B.Cu) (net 15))
 (segment (start 111.1 104.4) (end 111.1 102.41) (width 0.3) (layer B.Cu) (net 15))
 (segment (start 111.1 102.41) (end 109.96 101.27) (width 0.3) (layer B.Cu) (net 15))
 (segment (start 103.6 104.65) (end 103.6 104.6) (width 0.3) (layer B.Cu) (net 15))
 (segment (start 103.6 104.6) (end 104.4 103.8) (width 0.3) (layer B.Cu) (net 15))
 (segment (start 104.4 103.8) (end 107.45 103.8) (width 0.3) (layer B.Cu) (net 15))
 (segment (start 107.45 103.8) (end 107.7 104.05) (width 0.3) (layer B.Cu) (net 15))
 (segment (start 109.95 114.5) (end 109.95 113.75) (width 0.5) (layer B.Cu) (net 16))
 (segment (start 109.95 113.75) (end 109.6 113.4) (width 0.5) (layer B.Cu) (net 16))
 (segment (start 109.6 113.4) (end 107.4 113.4) (width 0.5) (layer B.Cu) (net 16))
 (segment (start 107.4 113.4) (end 107.2 113.2) (width 0.5) (layer B.Cu) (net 16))
 (segment (start 107.2 113.2) (end 106.2 113.2) (width 0.5) (layer B.Cu) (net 16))
 (segment (start 106.2 113.2) (end 105.8 112.8) (width 0.5) (layer B.Cu) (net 16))
 (segment (start 105.8 112.8) (end 105.8 109.1) (width 0.5) (layer B.Cu) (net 16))
 (segment (start 105.8 109.1) (end 106.3 108.6) (width 0.5) (layer B.Cu) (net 16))
 (segment (start 106.3 108.6) (end 108.2 108.6) (width 0.5) (layer B.Cu) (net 16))
 (segment (start 108.2 108.6) (end 109.4 109.8) (width 0.5) (layer B.Cu) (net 16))
 (segment (start 109.4 109.8) (end 113.6 109.8) (width 0.5) (layer B.Cu) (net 16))
 (segment (start 113.6 109.8) (end 114.6 108.8) (width 0.5) (layer B.Cu) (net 16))
 (segment (start 114.6 108.8) (end 114.6 107.4) (width 0.5) (layer B.Cu) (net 16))
 (segment (start 114.6 107.4) (end 116.6 105.4) (width 0.5) (layer B.Cu) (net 16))
 (segment (start 116.6 105.4) (end 116.6 102.83) (width 0.5) (layer B.Cu) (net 16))
 (segment (start 116.6 102.83) (end 115.04 101.27) (width 0.5) (layer B.Cu) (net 16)))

